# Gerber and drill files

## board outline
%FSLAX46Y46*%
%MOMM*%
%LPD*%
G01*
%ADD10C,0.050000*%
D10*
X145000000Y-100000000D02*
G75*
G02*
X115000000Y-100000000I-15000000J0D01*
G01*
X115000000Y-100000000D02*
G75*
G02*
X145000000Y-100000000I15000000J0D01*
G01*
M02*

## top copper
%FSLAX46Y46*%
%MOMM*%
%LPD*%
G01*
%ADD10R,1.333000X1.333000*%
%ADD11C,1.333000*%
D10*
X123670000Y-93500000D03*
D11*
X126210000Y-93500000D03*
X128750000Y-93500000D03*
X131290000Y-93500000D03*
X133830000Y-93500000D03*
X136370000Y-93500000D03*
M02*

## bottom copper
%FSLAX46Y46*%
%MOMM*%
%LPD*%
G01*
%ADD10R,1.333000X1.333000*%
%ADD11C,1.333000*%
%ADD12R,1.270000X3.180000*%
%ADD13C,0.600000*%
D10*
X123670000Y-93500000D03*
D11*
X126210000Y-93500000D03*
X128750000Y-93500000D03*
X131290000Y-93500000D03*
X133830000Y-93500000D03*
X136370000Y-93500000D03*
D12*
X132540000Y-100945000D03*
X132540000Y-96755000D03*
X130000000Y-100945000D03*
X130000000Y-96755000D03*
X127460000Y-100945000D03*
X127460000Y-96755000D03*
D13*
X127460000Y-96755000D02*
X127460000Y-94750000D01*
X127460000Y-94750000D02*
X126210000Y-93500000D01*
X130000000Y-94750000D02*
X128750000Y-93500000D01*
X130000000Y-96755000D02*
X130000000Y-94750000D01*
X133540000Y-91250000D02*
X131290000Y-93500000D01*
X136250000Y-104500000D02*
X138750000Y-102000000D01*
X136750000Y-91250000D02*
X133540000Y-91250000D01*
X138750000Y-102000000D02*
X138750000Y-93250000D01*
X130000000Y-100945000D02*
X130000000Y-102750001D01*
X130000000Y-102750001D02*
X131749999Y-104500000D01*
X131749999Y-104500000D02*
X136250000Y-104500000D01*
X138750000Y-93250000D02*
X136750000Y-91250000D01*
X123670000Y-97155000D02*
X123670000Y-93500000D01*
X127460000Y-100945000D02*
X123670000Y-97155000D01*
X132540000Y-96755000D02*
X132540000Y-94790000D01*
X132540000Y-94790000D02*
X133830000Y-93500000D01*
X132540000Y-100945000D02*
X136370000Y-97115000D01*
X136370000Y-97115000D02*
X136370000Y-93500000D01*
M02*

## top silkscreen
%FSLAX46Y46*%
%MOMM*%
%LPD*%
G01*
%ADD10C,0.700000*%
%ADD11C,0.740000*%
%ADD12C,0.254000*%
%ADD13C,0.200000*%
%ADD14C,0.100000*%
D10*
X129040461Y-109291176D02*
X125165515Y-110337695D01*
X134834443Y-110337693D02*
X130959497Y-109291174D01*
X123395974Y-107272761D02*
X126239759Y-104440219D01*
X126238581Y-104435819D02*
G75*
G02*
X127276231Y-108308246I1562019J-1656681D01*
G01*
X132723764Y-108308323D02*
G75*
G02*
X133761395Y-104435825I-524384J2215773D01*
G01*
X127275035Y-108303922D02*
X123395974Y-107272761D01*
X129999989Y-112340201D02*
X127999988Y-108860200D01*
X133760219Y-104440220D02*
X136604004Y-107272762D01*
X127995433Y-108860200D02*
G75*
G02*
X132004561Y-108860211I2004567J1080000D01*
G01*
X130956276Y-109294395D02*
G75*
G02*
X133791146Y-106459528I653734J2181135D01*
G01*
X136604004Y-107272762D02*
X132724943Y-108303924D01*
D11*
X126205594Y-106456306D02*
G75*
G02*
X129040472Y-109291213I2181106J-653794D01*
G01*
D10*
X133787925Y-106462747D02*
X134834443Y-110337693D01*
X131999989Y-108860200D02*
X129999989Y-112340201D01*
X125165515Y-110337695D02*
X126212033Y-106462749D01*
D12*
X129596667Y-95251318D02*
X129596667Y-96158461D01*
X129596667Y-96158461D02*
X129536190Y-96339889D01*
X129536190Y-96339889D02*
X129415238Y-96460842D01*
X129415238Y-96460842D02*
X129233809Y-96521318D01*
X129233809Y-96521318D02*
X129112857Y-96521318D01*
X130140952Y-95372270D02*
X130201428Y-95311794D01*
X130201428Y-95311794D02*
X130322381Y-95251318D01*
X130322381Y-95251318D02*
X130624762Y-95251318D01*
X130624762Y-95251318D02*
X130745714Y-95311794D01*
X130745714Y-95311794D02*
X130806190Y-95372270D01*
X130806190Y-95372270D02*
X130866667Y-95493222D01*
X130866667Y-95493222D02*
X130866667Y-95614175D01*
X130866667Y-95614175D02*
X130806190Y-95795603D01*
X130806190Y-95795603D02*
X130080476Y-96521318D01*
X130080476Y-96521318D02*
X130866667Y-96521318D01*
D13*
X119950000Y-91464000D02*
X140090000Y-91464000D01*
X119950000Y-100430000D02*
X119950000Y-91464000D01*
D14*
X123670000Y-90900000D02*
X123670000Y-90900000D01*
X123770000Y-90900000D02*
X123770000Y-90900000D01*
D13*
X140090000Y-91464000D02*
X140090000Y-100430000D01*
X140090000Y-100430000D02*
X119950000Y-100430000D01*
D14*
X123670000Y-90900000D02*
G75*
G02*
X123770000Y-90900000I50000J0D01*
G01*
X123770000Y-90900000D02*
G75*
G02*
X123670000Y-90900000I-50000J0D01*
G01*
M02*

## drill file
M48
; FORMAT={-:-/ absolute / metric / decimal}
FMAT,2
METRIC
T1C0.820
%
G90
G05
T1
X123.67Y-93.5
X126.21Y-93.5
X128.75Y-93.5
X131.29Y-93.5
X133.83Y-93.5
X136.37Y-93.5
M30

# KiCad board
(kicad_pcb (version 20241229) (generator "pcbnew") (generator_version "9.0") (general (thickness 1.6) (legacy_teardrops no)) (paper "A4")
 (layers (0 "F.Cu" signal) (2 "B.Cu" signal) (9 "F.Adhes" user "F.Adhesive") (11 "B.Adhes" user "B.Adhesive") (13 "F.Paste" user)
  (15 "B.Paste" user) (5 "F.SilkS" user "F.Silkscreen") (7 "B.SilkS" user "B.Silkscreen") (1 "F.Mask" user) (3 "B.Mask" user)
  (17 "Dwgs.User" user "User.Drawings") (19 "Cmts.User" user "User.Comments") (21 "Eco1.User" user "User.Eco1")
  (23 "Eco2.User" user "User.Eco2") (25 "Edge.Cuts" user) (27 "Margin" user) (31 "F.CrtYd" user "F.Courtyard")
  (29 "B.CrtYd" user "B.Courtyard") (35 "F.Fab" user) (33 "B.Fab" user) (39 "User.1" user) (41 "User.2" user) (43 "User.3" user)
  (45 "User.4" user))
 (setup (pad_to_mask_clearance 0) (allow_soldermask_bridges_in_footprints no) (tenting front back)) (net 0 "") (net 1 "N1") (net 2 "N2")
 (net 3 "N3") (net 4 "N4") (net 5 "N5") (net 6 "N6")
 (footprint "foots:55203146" (layer "F.Cu") (at 123.67 93.5)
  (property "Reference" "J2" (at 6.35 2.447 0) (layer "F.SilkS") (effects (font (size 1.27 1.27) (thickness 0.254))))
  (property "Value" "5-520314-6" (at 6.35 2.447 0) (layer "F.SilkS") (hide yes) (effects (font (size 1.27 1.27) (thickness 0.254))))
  (fp_line (start -3.72 -2.036) (end 16.42 -2.036) (stroke (width 0.2) (type solid)) (layer "F.SilkS"))
  (fp_line (start -3.72 6.93) (end -3.72 -2.036) (stroke (width 0.2) (type solid)) (layer "F.SilkS"))
  (fp_line (start 0 -2.6) (end 0 -2.6) (stroke (width 0.1) (type solid)) (layer "F.SilkS"))
  (fp_line (start 0.1 -2.6) (end 0.1 -2.6) (stroke (width 0.1) (type solid)) (layer "F.SilkS"))
  (fp_line (start 16.42 -2.036) (end 16.42 6.93) (stroke (width 0.2) (type solid)) (layer "F.SilkS"))
  (fp_line (start 16.42 6.93) (end -3.72 6.93) (stroke (width 0.2) (type solid)) (layer "F.SilkS"))
  (fp_arc (start 0 -2.6) (mid 0.05 -2.65) (end 0.1 -2.6) (stroke (width 0.1) (type solid)) (layer "F.SilkS"))
  (fp_arc (start 0.1 -2.6) (mid 0.05 -2.55) (end 0 -2.6) (stroke (width 0.1) (type solid)) (layer "F.SilkS"))
  (pad "1" thru_hole rect (at 0 0) (size 1.333 1.333) (drill 0.82) (layers "*.Cu" "*.Mask") (remove_unused_layers no) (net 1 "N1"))
  (pad "2" thru_hole circle (at 2.54 0) (size 1.333 1.333) (drill 0.82) (layers "*.Cu" "*.Mask") (remove_unused_layers no) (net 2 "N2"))
  (pad "3" thru_hole circle (at 5.08 0) (size 1.333 1.333) (drill 0.82) (layers "*.Cu" "*.Mask") (remove_unused_layers no) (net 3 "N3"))
  (pad "4" thru_hole circle (at 7.62 0) (size 1.333 1.333) (drill 0.82) (layers "*.Cu" "*.Mask") (remove_unused_layers no) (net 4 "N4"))
  (pad "5" thru_hole circle (at 10.16 0) (size 1.333 1.333) (drill 0.82) (layers "*.Cu" "*.Mask") (remove_unused_layers no) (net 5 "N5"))
  (pad "6" thru_hole circle (at 12.7 0) (size 1.333 1.333) (drill 0.82) (layers "*.Cu" "*.Mask") (remove_unused_layers no) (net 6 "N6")))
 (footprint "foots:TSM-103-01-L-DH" (layer "B.Cu") (at 130 105.25)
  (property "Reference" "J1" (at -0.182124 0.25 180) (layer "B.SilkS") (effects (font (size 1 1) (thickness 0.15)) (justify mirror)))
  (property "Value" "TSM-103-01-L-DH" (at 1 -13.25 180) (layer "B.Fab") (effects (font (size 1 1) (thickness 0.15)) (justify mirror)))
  (pad "01" smd rect (at 2.54 -4.305) (size 1.27 3.18) (layers "B.Cu" "B.Mask" "B.Paste") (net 6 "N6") (solder_mask_margin 0.102))
  (pad "02" smd rect (at 2.54 -8.495) (size 1.27 3.18) (layers "B.Cu" "B.Mask" "B.Paste") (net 5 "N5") (solder_mask_margin 0.102))
  (pad "03" smd rect (at 0 -4.305) (size 1.27 3.18) (layers "B.Cu" "B.Mask" "B.Paste") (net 4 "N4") (solder_mask_margin 0.102))
  (pad "04" smd rect (at 0 -8.495) (size 1.27 3.18) (layers "B.Cu" "B.Mask" "B.Paste") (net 3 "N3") (solder_mask_margin 0.102))
  (pad "05" smd rect (at -2.54 -4.305) (size 1.27 3.18) (layers "B.Cu" "B.Mask" "B.Paste") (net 1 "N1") (solder_mask_margin 0.102))
  (pad "06" smd rect (at -2.54 -8.495) (size 1.27 3.18) (layers "B.Cu" "B.Mask" "B.Paste") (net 2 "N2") (solder_mask_margin 0.102)))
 (gr_line (start 129.040461 109.291176) (end 125.165515 110.337695) (stroke (width 0.7) (type solid)) (layer "F.SilkS"))
 (gr_line (start 134.834443 110.337693) (end 130.959497 109.291174) (stroke (width 0.7) (type solid)) (layer "F.SilkS"))
 (gr_line (start 123.395974 107.272761) (end 126.239759 104.440219) (stroke (width 0.7) (type solid)) (layer "F.SilkS"))
 (gr_arc (start 126.238581 104.435819) (mid 130 105.503219) (end 127.276213 108.308322) (stroke (width 0.7) (type solid)) (layer "F.SilkS"))
 (gr_arc (start 132.723764 108.308323) (mid 129.999989 105.50322) (end 133.761399 104.435821) (stroke (width 0.7) (type solid))
  (layer "F.SilkS"))
 (gr_line (start 127.275035 108.303922) (end 123.395974 107.272761) (stroke (width 0.7) (type solid)) (layer "F.SilkS"))
 (gr_line (start 129.999989 112.340201) (end 127.999988 108.8602) (stroke (width 0.7) (type solid)) (layer "F.SilkS"))
 (gr_line (start 133.760219 104.44022) (end 136.604004 107.272762) (stroke (width 0.7) (type solid)) (layer "F.SilkS"))
 (gr_arc (start 127.995433 108.8602) (mid 129.999988 105.503221) (end 132.004543 108.860201) (stroke (width 0.7) (type solid))
  (layer "F.SilkS"))
 (gr_arc (start 130.956276 109.294395) (mid 129.999936 105.503183) (end 133.791146 106.459528) (stroke (width 0.7) (type solid))
  (layer "F.SilkS"))
 (gr_line (start 136.604004 107.272762) (end 132.724943 108.303924) (stroke (width 0.7) (type solid)) (layer "F.SilkS"))
 (gr_arc (start 126.205594 106.456306) (mid 129.99677 105.5) (end 129.040461 109.291176) (stroke (width 0.74) (type solid))
  (layer "F.SilkS"))
 (gr_line (start 133.787925 106.462747) (end 134.834443 110.337693) (stroke (width 0.7) (type solid)) (layer "F.SilkS"))
 (gr_line (start 131.999989 108.8602) (end 129.999989 112.340201) (stroke (width 0.7) (type solid)) (layer "F.SilkS"))
 (gr_line (start 125.165515 110.337695) (end 126.212033 106.462749) (stroke (width 0.7) (type solid)) (layer "F.SilkS"))
 (gr_circle (center 130 100) (end 145 100) (stroke (width 0.05) (type default)) (fill no) (layer "Edge.Cuts"))
 (segment (start 127.46 96.755) (end 127.46 94.75) (width 0.6) (layer "B.Cu") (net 2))
 (segment (start 127.46 94.75) (end 126.21 93.5) (width 0.6) (layer "B.Cu") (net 2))
 (segment (start 130 94.75) (end 128.75 93.5) (width 0.6) (layer "B.Cu") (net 3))
 (segment (start 130 96.755) (end 130 94.75) (width 0.6) (layer "B.Cu") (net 3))
 (segment (start 133.54 91.25) (end 131.29 93.5) (width 0.6) (layer "B.Cu") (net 4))
 (segment (start 136.25 104.5) (end 138.75 102) (width 0.6) (layer "B.Cu") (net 4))
 (segment (start 136.75 91.25) (end 133.54 91.25) (width 0.6) (layer "B.Cu") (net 4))
 (segment (start 138.75 102) (end 138.75 93.25) (width 0.6) (layer "B.Cu") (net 4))
 (segment (start 130 100.945) (end 130 102.750001) (width 0.6) (layer "B.Cu") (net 4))
 (segment (start 130 102.750001) (end 131.749999 104.5) (width 0.6) (layer "B.Cu") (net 4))
 (segment (start 131.749999 104.5) (end 136.25 104.5) (width 0.6) (layer "B.Cu") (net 4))
 (segment (start 138.75 93.25) (end 136.75 91.25) (width 0.6) (layer "B.Cu") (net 4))
 (segment (start 123.67 97.155) (end 123.67 93.5) (width 0.6) (layer "B.Cu") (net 1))
 (segment (start 127.46 100.945) (end 123.67 97.155) (width 0.6) (layer "B.Cu") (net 1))
 (segment (start 132.54 96.755) (end 132.54 94.79) (width 0.6) (layer "B.Cu") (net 5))
 (segment (start 132.54 94.79) (end 133.83 93.5) (width 0.6) (layer "B.Cu") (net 5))
 (segment (start 132.54 100.945) (end 136.37 97.115) (width 0.6) (layer "B.Cu") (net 6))
 (segment (start 136.37 97.115) (end 136.37 93.5) (width 0.6) (layer "B.Cu") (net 6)))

